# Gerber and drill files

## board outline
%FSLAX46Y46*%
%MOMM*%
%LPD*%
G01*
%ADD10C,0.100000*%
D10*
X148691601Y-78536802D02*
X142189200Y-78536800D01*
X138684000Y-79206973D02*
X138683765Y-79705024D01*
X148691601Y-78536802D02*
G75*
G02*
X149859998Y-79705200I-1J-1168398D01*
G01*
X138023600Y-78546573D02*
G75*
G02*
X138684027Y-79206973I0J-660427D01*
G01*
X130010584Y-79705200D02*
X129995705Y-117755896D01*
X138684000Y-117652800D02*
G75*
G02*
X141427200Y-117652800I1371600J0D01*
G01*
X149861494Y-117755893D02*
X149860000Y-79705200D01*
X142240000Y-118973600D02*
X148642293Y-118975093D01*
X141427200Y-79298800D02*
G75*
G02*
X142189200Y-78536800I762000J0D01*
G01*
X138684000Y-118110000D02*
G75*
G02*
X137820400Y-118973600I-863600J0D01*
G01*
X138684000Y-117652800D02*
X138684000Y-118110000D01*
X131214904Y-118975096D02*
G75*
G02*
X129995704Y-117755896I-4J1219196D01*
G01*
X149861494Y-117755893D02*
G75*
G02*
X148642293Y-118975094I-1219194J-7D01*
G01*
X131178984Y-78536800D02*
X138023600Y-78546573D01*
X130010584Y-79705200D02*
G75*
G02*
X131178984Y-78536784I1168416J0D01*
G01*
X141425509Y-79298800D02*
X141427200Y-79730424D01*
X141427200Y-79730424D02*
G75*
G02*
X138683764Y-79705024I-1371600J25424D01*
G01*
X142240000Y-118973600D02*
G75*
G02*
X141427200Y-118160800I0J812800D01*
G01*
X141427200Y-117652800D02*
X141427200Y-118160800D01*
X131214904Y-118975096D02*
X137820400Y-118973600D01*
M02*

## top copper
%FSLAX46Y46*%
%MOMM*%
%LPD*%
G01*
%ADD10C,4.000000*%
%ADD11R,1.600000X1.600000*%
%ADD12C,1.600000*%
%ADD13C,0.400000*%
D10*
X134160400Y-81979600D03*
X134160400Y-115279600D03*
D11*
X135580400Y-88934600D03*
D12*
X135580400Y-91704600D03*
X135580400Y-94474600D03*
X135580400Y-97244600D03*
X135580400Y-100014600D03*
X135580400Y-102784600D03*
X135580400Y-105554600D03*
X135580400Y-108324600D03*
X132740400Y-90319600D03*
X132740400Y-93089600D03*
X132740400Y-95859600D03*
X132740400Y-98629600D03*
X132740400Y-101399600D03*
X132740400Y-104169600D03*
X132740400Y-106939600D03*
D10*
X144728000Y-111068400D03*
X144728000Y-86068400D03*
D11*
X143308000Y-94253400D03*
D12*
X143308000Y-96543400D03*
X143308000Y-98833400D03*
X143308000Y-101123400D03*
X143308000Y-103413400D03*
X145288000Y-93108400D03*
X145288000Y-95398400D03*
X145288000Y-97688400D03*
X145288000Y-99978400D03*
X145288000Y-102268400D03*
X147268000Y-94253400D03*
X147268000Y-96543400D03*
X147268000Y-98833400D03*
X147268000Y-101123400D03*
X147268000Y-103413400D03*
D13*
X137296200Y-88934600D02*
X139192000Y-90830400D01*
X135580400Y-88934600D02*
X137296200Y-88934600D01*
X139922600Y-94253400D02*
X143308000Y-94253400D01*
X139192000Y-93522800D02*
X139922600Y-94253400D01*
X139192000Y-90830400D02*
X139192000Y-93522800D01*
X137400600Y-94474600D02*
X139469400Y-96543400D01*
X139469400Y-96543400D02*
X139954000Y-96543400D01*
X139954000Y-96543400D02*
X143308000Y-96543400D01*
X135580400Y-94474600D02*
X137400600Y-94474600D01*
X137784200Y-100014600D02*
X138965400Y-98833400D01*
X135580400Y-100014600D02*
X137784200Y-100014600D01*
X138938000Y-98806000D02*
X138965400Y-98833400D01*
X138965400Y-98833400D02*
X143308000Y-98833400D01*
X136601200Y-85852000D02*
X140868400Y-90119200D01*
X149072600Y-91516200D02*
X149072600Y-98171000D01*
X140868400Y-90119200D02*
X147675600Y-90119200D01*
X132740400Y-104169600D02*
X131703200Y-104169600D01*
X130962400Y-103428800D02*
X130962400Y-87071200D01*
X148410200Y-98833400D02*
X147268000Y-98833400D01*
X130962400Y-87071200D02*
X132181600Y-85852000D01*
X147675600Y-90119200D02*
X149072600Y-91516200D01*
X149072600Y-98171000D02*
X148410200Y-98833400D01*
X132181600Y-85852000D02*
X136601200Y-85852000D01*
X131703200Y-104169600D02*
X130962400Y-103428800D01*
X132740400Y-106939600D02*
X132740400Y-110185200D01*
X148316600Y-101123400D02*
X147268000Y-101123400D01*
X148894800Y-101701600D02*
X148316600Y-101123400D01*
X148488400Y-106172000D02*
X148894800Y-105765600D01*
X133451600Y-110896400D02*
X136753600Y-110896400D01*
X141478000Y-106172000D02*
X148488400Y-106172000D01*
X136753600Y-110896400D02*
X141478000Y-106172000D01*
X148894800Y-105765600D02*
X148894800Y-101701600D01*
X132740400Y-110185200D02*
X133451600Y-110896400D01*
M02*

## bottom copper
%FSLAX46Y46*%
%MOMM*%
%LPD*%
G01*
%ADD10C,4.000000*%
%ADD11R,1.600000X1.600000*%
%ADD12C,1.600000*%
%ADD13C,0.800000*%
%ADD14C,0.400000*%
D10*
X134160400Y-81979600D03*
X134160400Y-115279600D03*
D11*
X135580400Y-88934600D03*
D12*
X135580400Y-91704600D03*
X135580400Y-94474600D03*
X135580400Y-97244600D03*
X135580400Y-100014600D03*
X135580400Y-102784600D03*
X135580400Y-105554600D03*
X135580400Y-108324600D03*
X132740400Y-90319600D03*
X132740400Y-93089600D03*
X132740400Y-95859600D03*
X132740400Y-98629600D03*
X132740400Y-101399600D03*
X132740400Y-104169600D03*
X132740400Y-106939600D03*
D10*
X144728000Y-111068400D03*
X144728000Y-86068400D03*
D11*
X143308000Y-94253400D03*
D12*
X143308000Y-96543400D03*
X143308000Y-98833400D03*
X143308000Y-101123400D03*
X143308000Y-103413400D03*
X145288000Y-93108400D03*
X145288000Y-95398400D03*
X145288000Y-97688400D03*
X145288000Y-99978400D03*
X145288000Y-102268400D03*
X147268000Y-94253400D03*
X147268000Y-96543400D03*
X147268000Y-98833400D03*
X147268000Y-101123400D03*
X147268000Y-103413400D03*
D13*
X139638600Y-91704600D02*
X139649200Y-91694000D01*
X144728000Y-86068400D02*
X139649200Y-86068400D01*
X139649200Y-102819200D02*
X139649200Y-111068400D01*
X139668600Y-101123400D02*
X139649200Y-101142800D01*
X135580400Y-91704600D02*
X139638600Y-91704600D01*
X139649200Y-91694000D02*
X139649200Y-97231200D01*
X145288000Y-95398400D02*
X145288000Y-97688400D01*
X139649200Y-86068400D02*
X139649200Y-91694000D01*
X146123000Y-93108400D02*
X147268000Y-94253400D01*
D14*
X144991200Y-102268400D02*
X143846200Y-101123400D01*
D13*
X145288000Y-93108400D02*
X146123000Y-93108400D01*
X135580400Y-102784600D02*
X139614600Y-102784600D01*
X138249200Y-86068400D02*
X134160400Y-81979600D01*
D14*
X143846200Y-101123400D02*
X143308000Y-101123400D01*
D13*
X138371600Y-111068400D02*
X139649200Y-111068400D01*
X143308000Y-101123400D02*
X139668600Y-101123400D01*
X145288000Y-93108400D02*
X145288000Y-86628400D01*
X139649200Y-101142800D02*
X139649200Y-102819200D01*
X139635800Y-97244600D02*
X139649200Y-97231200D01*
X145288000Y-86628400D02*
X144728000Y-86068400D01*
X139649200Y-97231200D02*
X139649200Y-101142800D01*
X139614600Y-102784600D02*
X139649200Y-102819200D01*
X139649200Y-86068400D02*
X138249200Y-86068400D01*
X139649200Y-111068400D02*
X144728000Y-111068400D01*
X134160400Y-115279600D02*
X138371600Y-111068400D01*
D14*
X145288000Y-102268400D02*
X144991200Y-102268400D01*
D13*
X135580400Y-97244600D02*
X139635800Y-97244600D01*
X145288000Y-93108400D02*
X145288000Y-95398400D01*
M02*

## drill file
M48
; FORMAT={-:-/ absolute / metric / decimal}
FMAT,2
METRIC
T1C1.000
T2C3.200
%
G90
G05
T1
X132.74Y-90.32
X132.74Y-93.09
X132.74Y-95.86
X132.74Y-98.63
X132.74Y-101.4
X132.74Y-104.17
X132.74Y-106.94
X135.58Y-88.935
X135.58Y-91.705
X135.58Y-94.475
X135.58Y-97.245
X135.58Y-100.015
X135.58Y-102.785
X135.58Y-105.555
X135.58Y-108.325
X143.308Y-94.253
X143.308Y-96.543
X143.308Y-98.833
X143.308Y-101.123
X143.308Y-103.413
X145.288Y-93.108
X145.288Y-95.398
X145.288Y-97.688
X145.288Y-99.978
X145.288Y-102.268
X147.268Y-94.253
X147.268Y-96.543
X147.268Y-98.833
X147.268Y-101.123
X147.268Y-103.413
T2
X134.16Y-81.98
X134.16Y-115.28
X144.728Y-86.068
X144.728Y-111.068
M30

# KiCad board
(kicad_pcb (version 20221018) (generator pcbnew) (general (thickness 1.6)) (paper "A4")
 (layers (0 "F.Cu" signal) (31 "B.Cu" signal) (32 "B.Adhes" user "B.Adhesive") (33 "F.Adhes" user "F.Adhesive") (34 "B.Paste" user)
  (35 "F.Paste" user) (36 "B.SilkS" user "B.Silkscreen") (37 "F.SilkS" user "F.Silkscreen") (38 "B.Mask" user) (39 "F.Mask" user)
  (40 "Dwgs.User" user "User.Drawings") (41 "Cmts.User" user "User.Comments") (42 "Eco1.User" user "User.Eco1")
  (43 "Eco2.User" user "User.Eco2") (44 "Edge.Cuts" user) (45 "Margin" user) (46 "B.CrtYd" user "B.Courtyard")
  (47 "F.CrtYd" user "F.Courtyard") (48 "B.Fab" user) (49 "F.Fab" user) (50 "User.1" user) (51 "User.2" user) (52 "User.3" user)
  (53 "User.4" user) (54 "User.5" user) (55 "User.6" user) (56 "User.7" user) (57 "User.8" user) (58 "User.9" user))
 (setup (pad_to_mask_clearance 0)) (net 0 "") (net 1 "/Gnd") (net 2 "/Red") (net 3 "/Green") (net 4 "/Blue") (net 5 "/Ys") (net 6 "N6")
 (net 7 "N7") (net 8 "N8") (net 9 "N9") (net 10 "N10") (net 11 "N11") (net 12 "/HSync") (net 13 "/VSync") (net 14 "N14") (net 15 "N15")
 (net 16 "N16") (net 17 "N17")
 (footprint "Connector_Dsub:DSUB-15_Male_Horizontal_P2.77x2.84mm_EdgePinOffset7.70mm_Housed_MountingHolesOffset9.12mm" (layer "F.Cu")
  (at 135.5804 88.9346 -90)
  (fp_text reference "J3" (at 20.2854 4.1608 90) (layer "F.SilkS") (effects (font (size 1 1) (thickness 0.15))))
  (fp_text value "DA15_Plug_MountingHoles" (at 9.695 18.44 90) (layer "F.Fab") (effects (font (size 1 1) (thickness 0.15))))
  (pad "0" thru_hole circle (at -6.955 1.42 270) (size 4 4) (drill 3.2) (layers "*.Cu" "*.Mask") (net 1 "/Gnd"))
  (pad "0" thru_hole circle (at 26.345 1.42 270) (size 4 4) (drill 3.2) (layers "*.Cu" "*.Mask") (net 1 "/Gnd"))
  (pad "1" thru_hole rect (at 0 0 270) (size 1.6 1.6) (drill 1) (layers "*.Cu" "*.Mask") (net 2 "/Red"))
  (pad "2" thru_hole circle (at 2.77 0 270) (size 1.6 1.6) (drill 1) (layers "*.Cu" "*.Mask") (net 1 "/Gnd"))
  (pad "3" thru_hole circle (at 5.54 0 270) (size 1.6 1.6) (drill 1) (layers "*.Cu" "*.Mask") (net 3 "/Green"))
  (pad "4" thru_hole circle (at 8.31 0 270) (size 1.6 1.6) (drill 1) (layers "*.Cu" "*.Mask") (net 1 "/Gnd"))
  (pad "5" thru_hole circle (at 11.08 0 270) (size 1.6 1.6) (drill 1) (layers "*.Cu" "*.Mask") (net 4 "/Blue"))
  (pad "6" thru_hole circle (at 13.85 0 270) (size 1.6 1.6) (drill 1) (layers "*.Cu" "*.Mask") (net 1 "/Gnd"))
  (pad "7" thru_hole circle (at 16.62 0 270) (size 1.6 1.6) (drill 1) (layers "*.Cu" "*.Mask") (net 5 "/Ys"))
  (pad "8" thru_hole circle (at 19.39 0 270) (size 1.6 1.6) (drill 1) (layers "*.Cu" "*.Mask") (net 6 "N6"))
  (pad "9" thru_hole circle (at 1.385 2.84 270) (size 1.6 1.6) (drill 1) (layers "*.Cu" "*.Mask") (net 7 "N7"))
  (pad "10" thru_hole circle (at 4.155 2.84 270) (size 1.6 1.6) (drill 1) (layers "*.Cu" "*.Mask") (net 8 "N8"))
  (pad "11" thru_hole circle (at 6.925 2.84 270) (size 1.6 1.6) (drill 1) (layers "*.Cu" "*.Mask") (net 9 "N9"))
  (pad "12" thru_hole circle (at 9.695 2.84 270) (size 1.6 1.6) (drill 1) (layers "*.Cu" "*.Mask") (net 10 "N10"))
  (pad "13" thru_hole circle (at 12.465 2.84 270) (size 1.6 1.6) (drill 1) (layers "*.Cu" "*.Mask") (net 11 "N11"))
  (pad "14" thru_hole circle (at 15.235 2.84 270) (size 1.6 1.6) (drill 1) (layers "*.Cu" "*.Mask") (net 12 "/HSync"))
  (pad "15" thru_hole circle (at 18.005 2.84 270) (size 1.6 1.6) (drill 1) (layers "*.Cu" "*.Mask") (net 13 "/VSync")))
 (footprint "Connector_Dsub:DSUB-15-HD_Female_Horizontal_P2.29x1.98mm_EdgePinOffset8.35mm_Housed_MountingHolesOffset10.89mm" (layer "F.Cu")
  (at 143.308 94.2534 90)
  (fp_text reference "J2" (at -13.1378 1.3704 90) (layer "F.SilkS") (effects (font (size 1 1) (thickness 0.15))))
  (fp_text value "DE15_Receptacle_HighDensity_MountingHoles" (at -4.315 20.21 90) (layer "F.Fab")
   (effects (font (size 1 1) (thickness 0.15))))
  (pad "0" thru_hole circle (at -16.815 1.42 90) (size 4 4) (drill 3.2) (layers "*.Cu" "*.Mask") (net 1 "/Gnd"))
  (pad "0" thru_hole circle (at 8.185 1.42 90) (size 4 4) (drill 3.2) (layers "*.Cu" "*.Mask") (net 1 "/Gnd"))
  (pad "1" thru_hole rect (at 0 0 90) (size 1.6 1.6) (drill 1) (layers "*.Cu" "*.Mask") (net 2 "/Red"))
  (pad "2" thru_hole circle (at -2.29 0 90) (size 1.6 1.6) (drill 1) (layers "*.Cu" "*.Mask") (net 3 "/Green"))
  (pad "3" thru_hole circle (at -4.58 0 90) (size 1.6 1.6) (drill 1) (layers "*.Cu" "*.Mask") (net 4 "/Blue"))
  (pad "4" thru_hole circle (at -6.87 0 90) (size 1.6 1.6) (drill 1) (layers "*.Cu" "*.Mask") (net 1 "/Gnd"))
  (pad "5" thru_hole circle (at -9.16 0 90) (size 1.6 1.6) (drill 1) (layers "*.Cu" "*.Mask") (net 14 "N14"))
  (pad "6" thru_hole circle (at 1.145 1.98 90) (size 1.6 1.6) (drill 1) (layers "*.Cu" "*.Mask") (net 1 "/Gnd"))
  (pad "7" thru_hole circle (at -1.145 1.98 90) (size 1.6 1.6) (drill 1) (layers "*.Cu" "*.Mask") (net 1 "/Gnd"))
  (pad "8" thru_hole circle (at -3.435 1.98 90) (size 1.6 1.6) (drill 1) (layers "*.Cu" "*.Mask") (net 1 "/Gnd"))
  (pad "9" thru_hole circle (at -5.725 1.98 90) (size 1.6 1.6) (drill 1) (layers "*.Cu" "*.Mask") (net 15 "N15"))
  (pad "10" thru_hole circle (at -8.015 1.98 90) (size 1.6 1.6) (drill 1) (layers "*.Cu" "*.Mask") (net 1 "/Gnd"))
  (pad "11" thru_hole circle (at 0 3.96 90) (size 1.6 1.6) (drill 1) (layers "*.Cu" "*.Mask") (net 1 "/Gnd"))
  (pad "12" thru_hole circle (at -2.29 3.96 90) (size 1.6 1.6) (drill 1) (layers "*.Cu" "*.Mask") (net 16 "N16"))
  (pad "13" thru_hole circle (at -4.58 3.96 90) (size 1.6 1.6) (drill 1) (layers "*.Cu" "*.Mask") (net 12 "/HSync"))
  (pad "14" thru_hole circle (at -6.87 3.96 90) (size 1.6 1.6) (drill 1) (layers "*.Cu" "*.Mask") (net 13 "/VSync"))
  (pad "15" thru_hole circle (at -9.16 3.96 90) (size 1.6 1.6) (drill 1) (layers "*.Cu" "*.Mask") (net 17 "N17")))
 (gr_line (start 148.691601 78.536802) (end 142.1892 78.5368) (stroke (width 0.1) (type default)) (layer "Edge.Cuts"))
 (gr_line (start 138.684 79.206973) (end 138.683765 79.705024) (stroke (width 0.1) (type default)) (layer "Edge.Cuts"))
 (gr_arc (start 148.691601 78.536802) (mid 149.517772 78.879024) (end 149.86 79.7052) (stroke (width 0.1) (type default))
  (layer "Edge.Cuts"))
 (gr_arc (start 138.0236 78.546573) (mid 138.490573 78.74) (end 138.684 79.206973) (stroke (width 0.1) (type default)) (layer "Edge.Cuts"))
 (gr_line (start 130.010584 79.7052) (end 129.995705 117.755896) (stroke (width 0.1) (type default)) (layer "Edge.Cuts"))
 (gr_arc (start 138.684 117.6528) (mid 140.0556 116.2812) (end 141.4272 117.6528) (stroke (width 0.1) (type default)) (layer "Edge.Cuts"))
 (gr_line (start 149.861494 117.755893) (end 149.86 79.7052) (stroke (width 0.1) (type default)) (layer "Edge.Cuts"))
 (gr_line (start 142.24 118.9736) (end 148.642293 118.975093) (stroke (width 0.1) (type default)) (layer "Edge.Cuts"))
 (gr_arc (start 141.4272 79.2988) (mid 141.650385 78.759985) (end 142.1892 78.5368) (stroke (width 0.1) (type default)) (layer "Edge.Cuts"))
 (gr_arc (start 138.684 118.11) (mid 138.431057 118.720657) (end 137.8204 118.9736) (stroke (width 0.1) (type default)) (layer "Edge.Cuts"))
 (gr_line (start 138.684 117.6528) (end 138.684 118.11) (stroke (width 0.1) (type default)) (layer "Edge.Cuts"))
 (gr_arc (start 131.214904 118.975096) (mid 130.352798 118.618002) (end 129.995705 117.755896) (stroke (width 0.1) (type default))
  (layer "Edge.Cuts"))
 (gr_arc (start 149.861494 117.755893) (mid 149.5044 118.618) (end 148.642293 118.975093) (stroke (width 0.1) (type default))
  (layer "Edge.Cuts"))
 (gr_line (start 131.178984 78.5368) (end 138.0236 78.546573) (stroke (width 0.1) (type default)) (layer "Edge.Cuts"))
 (gr_arc (start 130.010584 79.7052) (mid 130.3528 78.879016) (end 131.178984 78.5368) (stroke (width 0.1) (type default))
  (layer "Edge.Cuts"))
 (gr_line (start 141.425509 79.2988) (end 141.4272 79.730424) (stroke (width 0.1) (type default)) (layer "Edge.Cuts"))
 (gr_arc (start 141.4272 79.730424) (mid 140.042899 81.0768) (end 138.683765 79.705024) (stroke (width 0.1) (type default))
  (layer "Edge.Cuts"))
 (gr_arc (start 142.24 118.9736) (mid 141.665264 118.735536) (end 141.4272 118.1608) (stroke (width 0.1) (type default)) (layer "Edge.Cuts"))
 (gr_line (start 141.4272 117.6528) (end 141.4272 118.1608) (stroke (width 0.1) (type default)) (layer "Edge.Cuts"))
 (gr_line (start 131.214904 118.975096) (end 137.8204 118.9736) (stroke (width 0.1) (type default)) (layer "Edge.Cuts"))
 (segment (start 139.6386 91.7046) (end 139.6492 91.694) (width 0.8) (layer "B.Cu") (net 1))
 (segment (start 144.728 86.0684) (end 139.6492 86.0684) (width 0.8) (layer "B.Cu") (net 1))
 (segment (start 139.6492 102.8192) (end 139.6492 111.0684) (width 0.8) (layer "B.Cu") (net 1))
 (segment (start 139.6686 101.1234) (end 139.6492 101.1428) (width 0.8) (layer "B.Cu") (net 1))
 (segment (start 135.5804 91.7046) (end 139.6386 91.7046) (width 0.8) (layer "B.Cu") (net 1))
 (segment (start 139.6492 91.694) (end 139.6492 97.2312) (width 0.8) (layer "B.Cu") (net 1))
 (segment (start 145.288 95.3984) (end 145.288 97.6884) (width 0.8) (layer "B.Cu") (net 1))
 (segment (start 139.6492 86.0684) (end 139.6492 91.694) (width 0.8) (layer "B.Cu") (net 1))
 (segment (start 146.123 93.1084) (end 147.268 94.2534) (width 0.8) (layer "B.Cu") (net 1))
 (segment (start 144.9912 102.2684) (end 143.8462 101.1234) (width 0.4) (layer "B.Cu") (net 1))
 (segment (start 145.288 93.1084) (end 146.123 93.1084) (width 0.8) (layer "B.Cu") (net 1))
 (segment (start 135.5804 102.7846) (end 139.6146 102.7846) (width 0.8) (layer "B.Cu") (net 1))
 (segment (start 138.2492 86.0684) (end 134.1604 81.9796) (width 0.8) (layer "B.Cu") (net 1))
 (segment (start 143.8462 101.1234) (end 143.308 101.1234) (width 0.4) (layer "B.Cu") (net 1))
 (segment (start 138.3716 111.0684) (end 139.6492 111.0684) (width 0.8) (layer "B.Cu") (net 1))
 (segment (start 143.308 101.1234) (end 139.6686 101.1234) (width 0.8) (layer "B.Cu") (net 1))
 (segment (start 145.288 93.1084) (end 145.288 86.6284) (width 0.8) (layer "B.Cu") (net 1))
 (segment (start 139.6492 101.1428) (end 139.6492 102.8192) (width 0.8) (layer "B.Cu") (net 1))
 (segment (start 139.6358 97.2446) (end 139.6492 97.2312) (width 0.8) (layer "B.Cu") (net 1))
 (segment (start 145.288 86.6284) (end 144.728 86.0684) (width 0.8) (layer "B.Cu") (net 1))
 (segment (start 139.6492 97.2312) (end 139.6492 101.1428) (width 0.8) (layer "B.Cu") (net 1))
 (segment (start 139.6146 102.7846) (end 139.6492 102.8192) (width 0.8) (layer "B.Cu") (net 1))
 (segment (start 139.6492 86.0684) (end 138.2492 86.0684) (width 0.8) (layer "B.Cu") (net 1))
 (segment (start 139.6492 111.0684) (end 144.728 111.0684) (width 0.8) (layer "B.Cu") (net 1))
 (segment (start 134.1604 115.2796) (end 138.3716 111.0684) (width 0.8) (layer "B.Cu") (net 1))
 (segment (start 145.288 102.2684) (end 144.9912 102.2684) (width 0.4) (layer "B.Cu") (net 1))
 (segment (start 135.5804 97.2446) (end 139.6358 97.2446) (width 0.8) (layer "B.Cu") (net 1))
 (segment (start 145.288 93.1084) (end 145.288 95.3984) (width 0.8) (layer "B.Cu") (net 1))
 (segment (start 137.2962 88.9346) (end 139.192 90.8304) (width 0.4) (layer "F.Cu") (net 2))
 (segment (start 135.5804 88.9346) (end 137.2962 88.9346) (width 0.4) (layer "F.Cu") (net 2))
 (segment (start 139.9226 94.2534) (end 143.308 94.2534) (width 0.4) (layer "F.Cu") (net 2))
 (segment (start 139.192 93.5228) (end 139.9226 94.2534) (width 0.4) (layer "F.Cu") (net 2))
 (segment (start 139.192 90.8304) (end 139.192 93.5228) (width 0.4) (layer "F.Cu") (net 2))
 (segment (start 137.4006 94.4746) (end 139.4694 96.5434) (width 0.4) (layer "F.Cu") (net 3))
 (segment (start 139.4694 96.5434) (end 139.954 96.5434) (width 0.4) (layer "F.Cu") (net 3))
 (segment (start 139.954 96.5434) (end 143.308 96.5434) (width 0.4) (layer "F.Cu") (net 3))
 (segment (start 135.5804 94.4746) (end 137.4006 94.4746) (width 0.4) (layer "F.Cu") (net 3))
 (segment (start 137.7842 100.0146) (end 138.9654 98.8334) (width 0.4) (layer "F.Cu") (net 4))
 (segment (start 135.5804 100.0146) (end 137.7842 100.0146) (width 0.4) (layer "F.Cu") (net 4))
 (segment (start 138.938 98.806) (end 138.9654 98.8334) (width 0.4) (layer "F.Cu") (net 4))
 (segment (start 138.9654 98.8334) (end 143.308 98.8334) (width 0.4) (layer "F.Cu") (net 4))
 (segment (start 136.6012 85.852) (end 140.8684 90.1192) (width 0.4) (layer "F.Cu") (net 12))
 (segment (start 149.0726 91.5162) (end 149.0726 98.171) (width 0.4) (layer "F.Cu") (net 12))
 (segment (start 140.8684 90.1192) (end 147.6756 90.1192) (width 0.4) (layer "F.Cu") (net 12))
 (segment (start 132.7404 104.1696) (end 131.7032 104.1696) (width 0.4) (layer "F.Cu") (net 12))
 (segment (start 130.9624 103.4288) (end 130.9624 87.0712) (width 0.4) (layer "F.Cu") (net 12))
 (segment (start 148.4102 98.8334) (end 147.268 98.8334) (width 0.4) (layer "F.Cu") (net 12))
 (segment (start 130.9624 87.0712) (end 132.1816 85.852) (width 0.4) (layer "F.Cu") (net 12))
 (segment (start 147.6756 90.1192) (end 149.0726 91.5162) (width 0.4) (layer "F.Cu") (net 12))
 (segment (start 149.0726 98.171) (end 148.4102 98.8334) (width 0.4) (layer "F.Cu") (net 12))
 (segment (start 132.1816 85.852) (end 136.6012 85.852) (width 0.4) (layer "F.Cu") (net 12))
 (segment (start 131.7032 104.1696) (end 130.9624 103.4288) (width 0.4) (layer "F.Cu") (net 12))
 (segment (start 132.7404 106.9396) (end 132.7404 110.1852) (width 0.4) (layer "F.Cu") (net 13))
 (segment (start 148.3166 101.1234) (end 147.268 101.1234) (width 0.4) (layer "F.Cu") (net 13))
 (segment (start 148.8948 101.7016) (end 148.3166 101.1234) (width 0.4) (layer "F.Cu") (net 13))
 (segment (start 148.4884 106.172) (end 148.8948 105.7656) (width 0.4) (layer "F.Cu") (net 13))
 (segment (start 133.4516 110.8964) (end 136.7536 110.8964) (width 0.4) (layer "F.Cu") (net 13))
 (segment (start 141.478 106.172) (end 148.4884 106.172) (width 0.4) (layer "F.Cu") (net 13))
 (segment (start 136.7536 110.8964) (end 141.478 106.172) (width 0.4) (layer "F.Cu") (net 13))
 (segment (start 148.8948 105.7656) (end 148.8948 101.7016) (width 0.4) (layer "F.Cu") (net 13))
 (segment (start 132.7404 110.1852) (end 133.4516 110.8964) (width 0.4) (layer "F.Cu") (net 13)))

